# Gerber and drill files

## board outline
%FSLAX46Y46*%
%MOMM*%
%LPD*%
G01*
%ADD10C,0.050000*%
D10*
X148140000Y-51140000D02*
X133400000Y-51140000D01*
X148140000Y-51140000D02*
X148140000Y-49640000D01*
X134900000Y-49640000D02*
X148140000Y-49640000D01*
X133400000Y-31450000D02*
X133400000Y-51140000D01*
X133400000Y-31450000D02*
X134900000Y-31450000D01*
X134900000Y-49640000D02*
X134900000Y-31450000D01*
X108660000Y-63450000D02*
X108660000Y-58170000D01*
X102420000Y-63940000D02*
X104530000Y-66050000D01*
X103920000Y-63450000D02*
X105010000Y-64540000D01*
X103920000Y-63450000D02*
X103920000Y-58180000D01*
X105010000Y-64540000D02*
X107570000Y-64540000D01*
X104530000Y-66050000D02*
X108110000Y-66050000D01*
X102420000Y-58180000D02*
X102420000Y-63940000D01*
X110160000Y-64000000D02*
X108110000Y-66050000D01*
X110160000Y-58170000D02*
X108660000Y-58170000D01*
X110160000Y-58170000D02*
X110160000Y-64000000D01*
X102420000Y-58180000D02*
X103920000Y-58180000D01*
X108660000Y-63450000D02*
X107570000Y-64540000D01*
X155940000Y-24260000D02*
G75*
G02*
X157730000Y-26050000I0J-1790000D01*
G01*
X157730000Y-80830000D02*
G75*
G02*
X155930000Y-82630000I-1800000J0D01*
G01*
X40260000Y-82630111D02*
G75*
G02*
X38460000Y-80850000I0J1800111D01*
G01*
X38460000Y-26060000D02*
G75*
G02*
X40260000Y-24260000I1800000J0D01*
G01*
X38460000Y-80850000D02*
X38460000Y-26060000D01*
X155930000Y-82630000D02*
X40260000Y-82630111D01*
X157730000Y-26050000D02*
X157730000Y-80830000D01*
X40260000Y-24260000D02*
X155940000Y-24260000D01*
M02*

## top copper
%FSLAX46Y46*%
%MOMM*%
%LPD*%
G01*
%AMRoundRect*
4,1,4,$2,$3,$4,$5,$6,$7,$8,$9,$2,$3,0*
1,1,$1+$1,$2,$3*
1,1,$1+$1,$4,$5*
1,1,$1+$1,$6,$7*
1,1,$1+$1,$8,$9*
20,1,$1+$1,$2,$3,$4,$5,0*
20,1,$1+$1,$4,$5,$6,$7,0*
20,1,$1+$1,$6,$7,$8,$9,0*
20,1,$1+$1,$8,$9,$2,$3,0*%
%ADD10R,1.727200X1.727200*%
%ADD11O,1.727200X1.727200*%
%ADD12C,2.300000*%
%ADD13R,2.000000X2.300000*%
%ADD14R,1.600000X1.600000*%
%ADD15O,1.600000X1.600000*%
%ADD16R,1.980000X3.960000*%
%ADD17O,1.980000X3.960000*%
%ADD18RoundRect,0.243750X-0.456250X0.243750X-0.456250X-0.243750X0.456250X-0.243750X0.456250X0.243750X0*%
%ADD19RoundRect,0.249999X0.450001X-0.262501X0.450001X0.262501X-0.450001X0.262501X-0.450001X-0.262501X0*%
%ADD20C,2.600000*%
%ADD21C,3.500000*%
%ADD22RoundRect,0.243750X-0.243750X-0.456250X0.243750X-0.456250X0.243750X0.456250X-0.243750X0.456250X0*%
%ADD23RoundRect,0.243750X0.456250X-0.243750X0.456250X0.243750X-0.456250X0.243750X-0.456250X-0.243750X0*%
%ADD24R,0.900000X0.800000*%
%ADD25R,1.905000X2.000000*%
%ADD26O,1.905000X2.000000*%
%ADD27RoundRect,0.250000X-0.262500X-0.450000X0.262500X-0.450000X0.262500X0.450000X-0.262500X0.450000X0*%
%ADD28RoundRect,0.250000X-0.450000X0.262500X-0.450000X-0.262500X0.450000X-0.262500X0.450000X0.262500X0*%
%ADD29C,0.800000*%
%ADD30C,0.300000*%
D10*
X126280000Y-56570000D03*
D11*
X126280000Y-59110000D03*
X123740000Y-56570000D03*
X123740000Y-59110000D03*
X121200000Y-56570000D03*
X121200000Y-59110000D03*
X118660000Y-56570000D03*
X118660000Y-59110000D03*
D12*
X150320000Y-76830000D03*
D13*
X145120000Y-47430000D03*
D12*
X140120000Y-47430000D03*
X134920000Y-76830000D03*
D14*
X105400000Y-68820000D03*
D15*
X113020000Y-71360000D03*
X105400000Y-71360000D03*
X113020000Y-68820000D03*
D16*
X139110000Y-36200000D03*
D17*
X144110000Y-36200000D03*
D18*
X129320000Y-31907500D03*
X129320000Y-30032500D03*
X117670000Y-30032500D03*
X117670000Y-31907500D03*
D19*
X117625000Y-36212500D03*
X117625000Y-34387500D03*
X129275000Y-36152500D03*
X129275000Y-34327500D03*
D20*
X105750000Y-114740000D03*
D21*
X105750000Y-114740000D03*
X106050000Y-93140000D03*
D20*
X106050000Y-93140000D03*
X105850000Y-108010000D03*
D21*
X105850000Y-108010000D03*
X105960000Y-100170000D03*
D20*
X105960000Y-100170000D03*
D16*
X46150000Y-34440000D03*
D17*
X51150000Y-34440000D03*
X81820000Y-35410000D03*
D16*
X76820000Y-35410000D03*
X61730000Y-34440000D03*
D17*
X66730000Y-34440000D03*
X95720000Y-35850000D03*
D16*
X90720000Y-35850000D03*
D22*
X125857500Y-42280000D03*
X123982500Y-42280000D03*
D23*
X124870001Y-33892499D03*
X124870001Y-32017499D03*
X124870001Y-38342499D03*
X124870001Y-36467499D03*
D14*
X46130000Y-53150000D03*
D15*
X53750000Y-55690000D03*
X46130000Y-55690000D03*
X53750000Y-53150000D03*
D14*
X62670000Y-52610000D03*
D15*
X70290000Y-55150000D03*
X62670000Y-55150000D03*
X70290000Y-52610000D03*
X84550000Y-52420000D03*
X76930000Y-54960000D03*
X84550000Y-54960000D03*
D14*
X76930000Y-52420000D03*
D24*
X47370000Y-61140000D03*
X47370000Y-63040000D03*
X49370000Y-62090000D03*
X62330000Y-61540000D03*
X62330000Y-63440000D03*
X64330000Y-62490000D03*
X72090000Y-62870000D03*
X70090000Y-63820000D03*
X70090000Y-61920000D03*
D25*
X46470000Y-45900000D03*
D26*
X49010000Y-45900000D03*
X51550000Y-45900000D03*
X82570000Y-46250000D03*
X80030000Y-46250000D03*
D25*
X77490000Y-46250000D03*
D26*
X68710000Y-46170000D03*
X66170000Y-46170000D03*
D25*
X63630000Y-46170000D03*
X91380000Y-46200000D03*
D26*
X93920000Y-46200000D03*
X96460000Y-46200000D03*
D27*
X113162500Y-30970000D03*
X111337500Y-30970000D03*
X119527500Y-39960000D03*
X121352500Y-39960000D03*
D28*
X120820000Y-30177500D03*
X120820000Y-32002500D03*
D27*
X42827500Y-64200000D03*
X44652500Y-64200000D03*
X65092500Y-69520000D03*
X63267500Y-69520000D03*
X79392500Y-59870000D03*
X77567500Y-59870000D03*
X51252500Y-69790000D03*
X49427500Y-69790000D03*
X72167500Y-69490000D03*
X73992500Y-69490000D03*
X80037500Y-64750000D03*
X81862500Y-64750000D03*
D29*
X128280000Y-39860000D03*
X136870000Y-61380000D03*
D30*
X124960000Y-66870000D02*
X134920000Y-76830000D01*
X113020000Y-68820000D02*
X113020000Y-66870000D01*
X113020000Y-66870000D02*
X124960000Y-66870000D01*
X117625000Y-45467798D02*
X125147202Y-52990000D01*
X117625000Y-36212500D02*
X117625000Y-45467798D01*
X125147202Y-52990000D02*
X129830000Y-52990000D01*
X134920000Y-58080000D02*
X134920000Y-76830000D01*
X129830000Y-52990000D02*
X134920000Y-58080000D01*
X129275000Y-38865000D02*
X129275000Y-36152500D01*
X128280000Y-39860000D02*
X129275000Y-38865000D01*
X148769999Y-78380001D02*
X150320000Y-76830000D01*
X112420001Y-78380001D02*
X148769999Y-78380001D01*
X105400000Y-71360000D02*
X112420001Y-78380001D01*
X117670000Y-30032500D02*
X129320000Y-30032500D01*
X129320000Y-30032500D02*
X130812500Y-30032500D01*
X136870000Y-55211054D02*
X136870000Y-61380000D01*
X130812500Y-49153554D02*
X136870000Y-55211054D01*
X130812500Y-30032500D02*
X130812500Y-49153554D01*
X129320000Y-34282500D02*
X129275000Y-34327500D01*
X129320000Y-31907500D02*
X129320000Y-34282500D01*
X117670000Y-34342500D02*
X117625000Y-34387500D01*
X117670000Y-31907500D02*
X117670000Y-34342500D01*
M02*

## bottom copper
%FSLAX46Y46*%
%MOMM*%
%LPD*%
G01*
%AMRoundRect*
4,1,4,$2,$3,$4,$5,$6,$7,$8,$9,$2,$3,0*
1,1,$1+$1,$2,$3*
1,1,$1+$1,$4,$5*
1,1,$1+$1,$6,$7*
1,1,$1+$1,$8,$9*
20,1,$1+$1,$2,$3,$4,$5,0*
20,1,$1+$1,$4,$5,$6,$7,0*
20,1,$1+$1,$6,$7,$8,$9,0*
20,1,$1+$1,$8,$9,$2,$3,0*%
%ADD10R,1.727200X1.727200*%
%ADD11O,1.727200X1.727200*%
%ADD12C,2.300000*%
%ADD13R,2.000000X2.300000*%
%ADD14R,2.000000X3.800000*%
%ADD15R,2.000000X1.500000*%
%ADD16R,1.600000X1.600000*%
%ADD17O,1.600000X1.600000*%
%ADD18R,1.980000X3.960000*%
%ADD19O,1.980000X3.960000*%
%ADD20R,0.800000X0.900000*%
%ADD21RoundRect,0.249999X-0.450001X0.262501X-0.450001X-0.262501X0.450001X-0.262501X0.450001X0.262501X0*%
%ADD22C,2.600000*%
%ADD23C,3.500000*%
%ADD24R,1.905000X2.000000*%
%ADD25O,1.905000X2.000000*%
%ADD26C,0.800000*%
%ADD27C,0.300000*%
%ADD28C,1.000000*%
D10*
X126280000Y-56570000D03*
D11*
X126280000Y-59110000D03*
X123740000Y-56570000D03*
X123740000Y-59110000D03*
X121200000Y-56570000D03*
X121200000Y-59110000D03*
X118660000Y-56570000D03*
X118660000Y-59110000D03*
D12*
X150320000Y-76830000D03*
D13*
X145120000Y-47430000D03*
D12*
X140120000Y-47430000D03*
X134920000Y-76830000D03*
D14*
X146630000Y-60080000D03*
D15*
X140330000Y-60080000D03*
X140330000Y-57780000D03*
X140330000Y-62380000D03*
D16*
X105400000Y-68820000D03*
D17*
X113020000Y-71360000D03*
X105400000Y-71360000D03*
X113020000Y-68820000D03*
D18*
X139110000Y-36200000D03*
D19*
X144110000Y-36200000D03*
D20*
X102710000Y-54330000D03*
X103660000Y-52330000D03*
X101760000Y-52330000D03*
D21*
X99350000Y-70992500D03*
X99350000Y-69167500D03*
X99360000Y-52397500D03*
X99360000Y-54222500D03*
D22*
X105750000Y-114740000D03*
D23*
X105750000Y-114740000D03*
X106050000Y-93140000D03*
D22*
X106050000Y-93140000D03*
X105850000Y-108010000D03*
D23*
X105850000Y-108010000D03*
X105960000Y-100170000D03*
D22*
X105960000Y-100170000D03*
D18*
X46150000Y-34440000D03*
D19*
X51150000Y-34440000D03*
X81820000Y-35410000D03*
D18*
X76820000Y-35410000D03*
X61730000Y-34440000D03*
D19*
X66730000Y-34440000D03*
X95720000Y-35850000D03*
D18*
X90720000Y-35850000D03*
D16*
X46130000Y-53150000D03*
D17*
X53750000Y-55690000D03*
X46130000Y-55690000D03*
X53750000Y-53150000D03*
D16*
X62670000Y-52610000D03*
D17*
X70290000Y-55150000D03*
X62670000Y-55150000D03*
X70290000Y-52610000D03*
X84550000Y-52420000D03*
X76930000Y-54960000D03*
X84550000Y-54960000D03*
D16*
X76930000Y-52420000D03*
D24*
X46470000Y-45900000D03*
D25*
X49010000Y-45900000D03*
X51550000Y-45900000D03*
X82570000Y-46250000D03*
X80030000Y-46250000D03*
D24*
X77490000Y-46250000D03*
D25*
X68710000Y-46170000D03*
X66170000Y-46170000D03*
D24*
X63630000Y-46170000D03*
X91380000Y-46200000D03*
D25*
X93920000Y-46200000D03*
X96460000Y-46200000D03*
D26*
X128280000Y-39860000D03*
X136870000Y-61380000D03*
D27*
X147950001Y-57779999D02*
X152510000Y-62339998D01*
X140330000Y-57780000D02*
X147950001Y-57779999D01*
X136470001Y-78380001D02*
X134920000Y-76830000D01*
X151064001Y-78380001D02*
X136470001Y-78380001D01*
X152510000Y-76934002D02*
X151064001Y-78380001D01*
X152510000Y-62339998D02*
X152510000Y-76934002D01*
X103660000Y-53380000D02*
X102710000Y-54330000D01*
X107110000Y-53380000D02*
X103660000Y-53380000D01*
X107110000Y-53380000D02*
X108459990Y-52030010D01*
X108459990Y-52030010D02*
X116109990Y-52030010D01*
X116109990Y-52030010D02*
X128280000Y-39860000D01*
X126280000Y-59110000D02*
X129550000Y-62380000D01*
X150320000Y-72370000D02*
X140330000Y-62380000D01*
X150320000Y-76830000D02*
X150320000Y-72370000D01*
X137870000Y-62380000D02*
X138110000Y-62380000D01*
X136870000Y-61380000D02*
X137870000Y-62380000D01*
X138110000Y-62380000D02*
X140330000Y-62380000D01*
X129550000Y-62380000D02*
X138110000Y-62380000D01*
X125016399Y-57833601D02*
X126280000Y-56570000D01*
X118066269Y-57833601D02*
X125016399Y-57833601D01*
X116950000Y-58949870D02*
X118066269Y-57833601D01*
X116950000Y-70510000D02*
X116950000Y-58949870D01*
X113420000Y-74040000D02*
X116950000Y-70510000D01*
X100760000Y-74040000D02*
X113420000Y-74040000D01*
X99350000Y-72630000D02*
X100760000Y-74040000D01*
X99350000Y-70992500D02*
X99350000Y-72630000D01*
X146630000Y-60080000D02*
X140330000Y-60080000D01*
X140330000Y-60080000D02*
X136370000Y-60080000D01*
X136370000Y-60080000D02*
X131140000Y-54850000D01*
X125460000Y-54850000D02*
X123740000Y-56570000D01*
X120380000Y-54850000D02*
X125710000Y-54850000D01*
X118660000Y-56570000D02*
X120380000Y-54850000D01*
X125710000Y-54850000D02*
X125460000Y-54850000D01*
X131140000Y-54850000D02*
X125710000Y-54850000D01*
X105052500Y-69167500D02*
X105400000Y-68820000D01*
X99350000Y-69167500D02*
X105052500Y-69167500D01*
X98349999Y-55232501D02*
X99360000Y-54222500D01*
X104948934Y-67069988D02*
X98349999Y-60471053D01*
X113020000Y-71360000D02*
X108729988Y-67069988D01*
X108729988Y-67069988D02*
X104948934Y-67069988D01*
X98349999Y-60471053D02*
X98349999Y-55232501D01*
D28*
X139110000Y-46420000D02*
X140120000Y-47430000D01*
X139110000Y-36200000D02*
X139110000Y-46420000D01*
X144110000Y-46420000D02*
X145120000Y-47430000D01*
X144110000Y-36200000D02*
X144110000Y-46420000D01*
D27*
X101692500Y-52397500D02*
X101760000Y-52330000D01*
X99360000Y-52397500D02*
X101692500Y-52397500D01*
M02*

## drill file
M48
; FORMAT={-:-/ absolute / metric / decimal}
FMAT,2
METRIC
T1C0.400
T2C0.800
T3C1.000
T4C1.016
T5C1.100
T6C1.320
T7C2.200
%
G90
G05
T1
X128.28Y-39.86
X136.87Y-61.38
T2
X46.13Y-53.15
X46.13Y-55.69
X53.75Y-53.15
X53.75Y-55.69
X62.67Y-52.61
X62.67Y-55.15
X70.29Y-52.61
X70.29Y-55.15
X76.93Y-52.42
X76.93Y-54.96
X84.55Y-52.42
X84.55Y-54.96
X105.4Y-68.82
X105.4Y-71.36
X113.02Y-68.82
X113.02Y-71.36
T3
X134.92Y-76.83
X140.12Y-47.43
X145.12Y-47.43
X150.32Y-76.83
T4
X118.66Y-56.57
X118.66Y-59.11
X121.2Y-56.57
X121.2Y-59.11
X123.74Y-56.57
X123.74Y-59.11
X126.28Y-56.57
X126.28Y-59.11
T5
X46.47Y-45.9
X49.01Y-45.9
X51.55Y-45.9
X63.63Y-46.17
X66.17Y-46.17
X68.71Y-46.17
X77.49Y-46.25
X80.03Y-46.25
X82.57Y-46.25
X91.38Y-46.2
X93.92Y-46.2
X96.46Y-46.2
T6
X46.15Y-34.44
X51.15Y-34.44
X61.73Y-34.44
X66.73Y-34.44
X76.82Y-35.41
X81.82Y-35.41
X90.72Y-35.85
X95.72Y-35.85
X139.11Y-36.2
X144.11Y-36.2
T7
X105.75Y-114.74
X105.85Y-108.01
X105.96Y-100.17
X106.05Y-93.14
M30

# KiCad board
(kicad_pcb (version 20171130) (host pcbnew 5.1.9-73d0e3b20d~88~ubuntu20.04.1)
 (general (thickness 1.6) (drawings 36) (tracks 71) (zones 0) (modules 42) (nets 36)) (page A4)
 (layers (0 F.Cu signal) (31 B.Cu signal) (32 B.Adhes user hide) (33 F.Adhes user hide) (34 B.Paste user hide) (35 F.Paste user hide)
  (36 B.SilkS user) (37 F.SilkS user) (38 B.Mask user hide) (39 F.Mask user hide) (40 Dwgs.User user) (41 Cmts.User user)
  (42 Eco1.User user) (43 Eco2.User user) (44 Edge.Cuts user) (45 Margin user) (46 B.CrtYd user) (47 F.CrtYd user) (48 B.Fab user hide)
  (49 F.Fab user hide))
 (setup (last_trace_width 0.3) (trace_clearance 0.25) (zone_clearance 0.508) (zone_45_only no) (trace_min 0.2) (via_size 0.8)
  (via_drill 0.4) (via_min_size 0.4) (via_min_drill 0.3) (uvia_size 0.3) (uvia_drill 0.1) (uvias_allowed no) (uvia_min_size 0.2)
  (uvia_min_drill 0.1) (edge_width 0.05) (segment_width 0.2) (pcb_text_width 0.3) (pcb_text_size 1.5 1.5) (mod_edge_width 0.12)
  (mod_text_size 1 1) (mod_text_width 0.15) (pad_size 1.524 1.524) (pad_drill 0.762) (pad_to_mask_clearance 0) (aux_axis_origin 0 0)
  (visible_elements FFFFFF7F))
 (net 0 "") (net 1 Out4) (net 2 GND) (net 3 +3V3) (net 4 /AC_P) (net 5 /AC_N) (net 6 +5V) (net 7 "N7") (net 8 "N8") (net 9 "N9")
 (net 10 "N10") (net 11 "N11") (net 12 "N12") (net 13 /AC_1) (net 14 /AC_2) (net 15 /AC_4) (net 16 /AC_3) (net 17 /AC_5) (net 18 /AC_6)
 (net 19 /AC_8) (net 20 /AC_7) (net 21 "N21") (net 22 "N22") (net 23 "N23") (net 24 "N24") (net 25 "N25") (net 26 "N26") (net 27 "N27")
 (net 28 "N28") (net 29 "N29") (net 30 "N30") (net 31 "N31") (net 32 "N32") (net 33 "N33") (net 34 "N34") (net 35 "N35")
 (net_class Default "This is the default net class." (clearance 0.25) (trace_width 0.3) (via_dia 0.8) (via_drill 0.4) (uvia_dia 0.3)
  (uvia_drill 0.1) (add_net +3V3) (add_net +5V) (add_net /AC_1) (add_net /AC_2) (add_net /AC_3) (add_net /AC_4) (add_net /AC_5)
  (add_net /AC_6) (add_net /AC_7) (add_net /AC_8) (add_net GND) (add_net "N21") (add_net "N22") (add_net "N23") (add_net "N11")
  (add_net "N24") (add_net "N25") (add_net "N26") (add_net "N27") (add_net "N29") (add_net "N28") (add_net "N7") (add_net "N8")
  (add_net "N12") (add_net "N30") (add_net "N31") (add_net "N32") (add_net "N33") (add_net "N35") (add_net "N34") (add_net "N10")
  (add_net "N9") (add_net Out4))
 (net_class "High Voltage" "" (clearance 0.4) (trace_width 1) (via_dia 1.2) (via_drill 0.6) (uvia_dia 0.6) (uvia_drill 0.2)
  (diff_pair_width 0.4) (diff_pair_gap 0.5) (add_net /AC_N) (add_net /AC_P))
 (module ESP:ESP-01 (layer F.Cu) (at 126.28 56.57 270)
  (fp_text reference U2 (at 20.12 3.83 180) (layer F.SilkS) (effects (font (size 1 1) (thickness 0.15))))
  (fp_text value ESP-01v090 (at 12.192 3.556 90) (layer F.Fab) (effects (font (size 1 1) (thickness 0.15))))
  (pad 1 thru_hole rect (at 0 0 270) (size 1.7272 1.7272) (drill 1.016) (layers *.Cu *.Mask F.SilkS) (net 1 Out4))
  (pad 2 thru_hole oval (at 2.54 0 270) (size 1.7272 1.7272) (drill 1.016) (layers *.Cu *.Mask F.SilkS) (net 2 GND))
  (pad 3 thru_hole oval (at 0 2.54 270) (size 1.7272 1.7272) (drill 1.016) (layers *.Cu *.Mask F.SilkS) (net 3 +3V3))
  (pad 4 thru_hole oval (at 2.54 2.54 270) (size 1.7272 1.7272) (drill 1.016) (layers *.Cu *.Mask F.SilkS))
  (pad 5 thru_hole oval (at 0 5.08 270) (size 1.7272 1.7272) (drill 1.016) (layers *.Cu *.Mask F.SilkS))
  (pad 6 thru_hole oval (at 2.54 5.08 270) (size 1.7272 1.7272) (drill 1.016) (layers *.Cu *.Mask F.SilkS))
  (pad 7 thru_hole oval (at 0 7.62 270) (size 1.7272 1.7272) (drill 1.016) (layers *.Cu *.Mask F.SilkS) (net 3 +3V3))
  (pad 8 thru_hole oval (at 2.54 7.62 270) (size 1.7272 1.7272) (drill 1.016) (layers *.Cu *.Mask F.SilkS)))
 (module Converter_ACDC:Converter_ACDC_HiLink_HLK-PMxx (layer F.Cu) (at 145.12 47.43 270)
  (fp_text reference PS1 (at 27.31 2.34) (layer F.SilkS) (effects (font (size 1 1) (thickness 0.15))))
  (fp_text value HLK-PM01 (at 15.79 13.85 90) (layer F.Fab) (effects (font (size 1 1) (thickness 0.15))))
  (pad 3 thru_hole circle (at 29.4 -5.2 270) (size 2.3 2.3) (drill 1) (layers *.Cu *.Mask) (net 2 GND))
  (pad 1 thru_hole rect (at 0 0 270) (size 2.3 2) (drill 1) (layers *.Cu *.Mask) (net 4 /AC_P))
  (pad 2 thru_hole circle (at 0 5 270) (size 2.3 2.3) (drill 1) (layers *.Cu *.Mask) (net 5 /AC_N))
  (pad 4 thru_hole circle (at 29.4 10.2 270) (size 2.3 2.3) (drill 1) (layers *.Cu *.Mask) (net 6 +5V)))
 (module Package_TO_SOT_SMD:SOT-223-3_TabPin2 (layer B.Cu) (at 143.48 60.08)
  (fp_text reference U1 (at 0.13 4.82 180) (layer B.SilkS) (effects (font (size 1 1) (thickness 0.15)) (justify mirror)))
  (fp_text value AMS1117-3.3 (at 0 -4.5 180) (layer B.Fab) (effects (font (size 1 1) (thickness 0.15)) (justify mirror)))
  (pad 2 smd rect (at 3.15 0) (size 2 3.8) (layers B.Cu B.Paste B.Mask) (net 3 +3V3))
  (pad 2 smd rect (at -3.15 0) (size 2 1.5) (layers B.Cu B.Paste B.Mask) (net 3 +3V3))
  (pad 3 smd rect (at -3.15 -2.3) (size 2 1.5) (layers B.Cu B.Paste B.Mask) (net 6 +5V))
  (pad 1 smd rect (at -3.15 2.3) (size 2 1.5) (layers B.Cu B.Paste B.Mask) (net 2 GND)))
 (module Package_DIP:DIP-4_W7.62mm (layer F.Cu) (at 105.4 68.82)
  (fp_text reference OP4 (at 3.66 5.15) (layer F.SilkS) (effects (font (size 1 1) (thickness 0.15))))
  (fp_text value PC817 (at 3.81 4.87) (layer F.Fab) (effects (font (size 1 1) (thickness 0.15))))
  (pad 1 thru_hole rect (at 0 0) (size 1.6 1.6) (drill 0.8) (layers *.Cu *.Mask) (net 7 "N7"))
  (pad 3 thru_hole oval (at 7.62 2.54) (size 1.6 1.6) (drill 0.8) (layers *.Cu *.Mask) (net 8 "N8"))
  (pad 2 thru_hole oval (at 0 2.54) (size 1.6 1.6) (drill 0.8) (layers *.Cu *.Mask) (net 2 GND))
  (pad 4 thru_hole oval (at 7.62 0) (size 1.6 1.6) (drill 0.8) (layers *.Cu *.Mask) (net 6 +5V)))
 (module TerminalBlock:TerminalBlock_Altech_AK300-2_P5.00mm (layer F.Cu) (at 139.11 36.2)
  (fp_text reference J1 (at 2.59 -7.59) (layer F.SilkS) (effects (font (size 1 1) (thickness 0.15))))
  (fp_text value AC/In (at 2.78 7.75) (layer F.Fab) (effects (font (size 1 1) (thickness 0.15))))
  (pad 1 thru_hole rect (at 0 0) (size 1.98 3.96) (drill 1.32) (layers *.Cu *.Mask) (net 5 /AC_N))
  (pad 2 thru_hole oval (at 5 0) (size 1.98 3.96) (drill 1.32) (layers *.Cu *.Mask) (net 4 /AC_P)))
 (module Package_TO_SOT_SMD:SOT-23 (layer B.Cu) (at 102.71 53.33 270)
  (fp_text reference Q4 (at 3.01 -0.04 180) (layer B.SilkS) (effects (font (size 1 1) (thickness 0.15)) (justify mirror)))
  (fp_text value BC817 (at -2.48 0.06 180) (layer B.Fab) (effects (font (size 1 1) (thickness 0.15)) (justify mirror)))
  (pad 3 smd rect (at 1 0 270) (size 0.9 0.8) (layers B.Cu B.Paste B.Mask) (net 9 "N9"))
  (pad 2 smd rect (at -1 -0.95 270) (size 0.9 0.8) (layers B.Cu B.Paste B.Mask) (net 2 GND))
  (pad 1 smd rect (at -1 0.95 270) (size 0.9 0.8) (layers B.Cu B.Paste B.Mask) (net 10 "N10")))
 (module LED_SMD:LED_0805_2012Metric (layer F.Cu) (at 129.32 30.97 270)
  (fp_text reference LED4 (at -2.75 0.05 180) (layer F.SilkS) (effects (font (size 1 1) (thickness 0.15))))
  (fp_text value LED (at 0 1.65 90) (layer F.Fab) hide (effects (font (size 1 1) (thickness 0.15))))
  (pad 2 smd roundrect (at 0.9375 0 270) (size 0.975 1.4) (layers F.Cu F.Paste F.Mask) (roundrect_rratio 0.25) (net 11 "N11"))
  (pad 1 smd roundrect (at -0.9375 0 270) (size 0.975 1.4) (layers F.Cu F.Paste F.Mask) (roundrect_rratio 0.25) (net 2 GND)))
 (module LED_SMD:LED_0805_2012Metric (layer F.Cu) (at 117.67 30.97 270)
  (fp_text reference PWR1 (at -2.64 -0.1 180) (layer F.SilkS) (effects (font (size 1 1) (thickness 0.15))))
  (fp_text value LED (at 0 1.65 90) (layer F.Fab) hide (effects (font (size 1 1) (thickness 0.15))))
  (pad 1 smd roundrect (at -0.9375 0 270) (size 0.975 1.4) (layers F.Cu F.Paste F.Mask) (roundrect_rratio 0.25) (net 2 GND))
  (pad 2 smd roundrect (at 0.9375 0 270) (size 0.975 1.4) (layers F.Cu F.Paste F.Mask) (roundrect_rratio 0.25) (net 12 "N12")))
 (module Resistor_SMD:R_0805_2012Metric (layer F.Cu) (at 117.625 35.3 90)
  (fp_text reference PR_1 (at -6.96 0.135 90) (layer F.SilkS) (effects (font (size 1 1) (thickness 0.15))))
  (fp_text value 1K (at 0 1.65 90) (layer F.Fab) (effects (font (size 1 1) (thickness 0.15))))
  (pad 1 smd roundrect (at -0.9125 0 90) (size 1.025 1.4) (layers F.Cu F.Paste F.Mask) (roundrect_rratio 0.2439014634146341) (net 6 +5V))
  (pad 2 smd roundrect (at 0.9125 0 90) (size 1.025 1.4) (layers F.Cu F.Paste F.Mask) (roundrect_rratio 0.2439014634146341) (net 12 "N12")))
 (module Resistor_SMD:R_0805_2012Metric (layer F.Cu) (at 129.275 35.24 90)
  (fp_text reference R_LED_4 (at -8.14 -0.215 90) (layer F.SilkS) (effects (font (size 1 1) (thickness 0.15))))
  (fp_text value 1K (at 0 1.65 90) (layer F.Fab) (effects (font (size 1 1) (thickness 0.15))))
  (pad 1 smd roundrect (at -0.9125 0 90) (size 1.025 1.4) (layers F.Cu F.Paste F.Mask) (roundrect_rratio 0.2439014634146341) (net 9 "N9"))
  (pad 2 smd roundrect (at 0.9125 0 90) (size 1.025 1.4) (layers F.Cu F.Paste F.Mask) (roundrect_rratio 0.2439014634146341) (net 11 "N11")))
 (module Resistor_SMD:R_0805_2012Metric (layer B.Cu) (at 99.35 70.08 270)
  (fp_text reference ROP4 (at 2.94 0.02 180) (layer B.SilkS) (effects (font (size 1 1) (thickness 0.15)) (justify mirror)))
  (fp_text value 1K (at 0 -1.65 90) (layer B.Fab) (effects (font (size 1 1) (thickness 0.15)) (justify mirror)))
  (pad 2 smd roundrect (at 0.9125 0 270) (size 1.025 1.4) (layers B.Cu B.Paste B.Mask) (roundrect_rratio 0.2439014634146341) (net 1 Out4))
  (pad 1 smd roundrect (at -0.9125 0 270) (size 1.025 1.4) (layers B.Cu B.Paste B.Mask) (roundrect_rratio 0.2439014634146341) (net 7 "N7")))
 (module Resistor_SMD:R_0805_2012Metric (layer B.Cu) (at 99.36 53.31 270)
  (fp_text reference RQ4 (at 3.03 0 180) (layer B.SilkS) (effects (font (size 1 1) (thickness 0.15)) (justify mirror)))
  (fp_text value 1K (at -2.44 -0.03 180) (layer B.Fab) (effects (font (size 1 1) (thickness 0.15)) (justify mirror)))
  (pad 1 smd roundrect (at -0.9125 0 270) (size 1.025 1.4) (layers B.Cu B.Paste B.Mask) (roundrect_rratio 0.2439014634146341) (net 10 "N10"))
  (pad 2 smd roundrect (at 0.9125 0 270) (size 1.025 1.4) (layers B.Cu B.Paste B.Mask) (roundrect_rratio 0.2439014634146341) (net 8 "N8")))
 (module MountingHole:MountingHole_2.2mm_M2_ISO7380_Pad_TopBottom (layer F.Cu) (at 105.75 114.74)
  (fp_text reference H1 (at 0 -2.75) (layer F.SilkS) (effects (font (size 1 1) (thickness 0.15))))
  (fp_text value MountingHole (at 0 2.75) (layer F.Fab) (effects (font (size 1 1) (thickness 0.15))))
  (pad 1 thru_hole circle (at 0 0) (size 2.6 2.6) (drill 2.2) (layers *.Cu *.Mask))
  (pad 1 connect circle (at 0 0) (size 3.5 3.5) (layers F.Cu F.Mask))
  (pad 1 connect circle (at 0 0) (size 3.5 3.5) (layers B.Cu B.Mask)))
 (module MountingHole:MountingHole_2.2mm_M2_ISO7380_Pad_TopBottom (layer F.Cu) (at 106.05 93.14)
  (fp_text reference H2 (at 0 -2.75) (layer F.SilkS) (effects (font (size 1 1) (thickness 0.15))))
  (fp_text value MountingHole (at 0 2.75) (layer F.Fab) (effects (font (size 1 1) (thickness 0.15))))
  (pad 1 connect circle (at 0 0) (size 3.5 3.5) (layers B.Cu B.Mask))
  (pad 1 connect circle (at 0 0) (size 3.5 3.5) (layers F.Cu F.Mask))
  (pad 1 thru_hole circle (at 0 0) (size 2.6 2.6) (drill 2.2) (layers *.Cu *.Mask)))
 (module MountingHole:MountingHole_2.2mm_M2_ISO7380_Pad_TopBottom (layer F.Cu) (at 105.85 108.01)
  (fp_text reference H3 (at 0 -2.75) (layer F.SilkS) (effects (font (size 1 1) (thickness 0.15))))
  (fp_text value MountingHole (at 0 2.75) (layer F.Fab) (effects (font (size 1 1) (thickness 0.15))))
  (pad 1 thru_hole circle (at 0 0) (size 2.6 2.6) (drill 2.2) (layers *.Cu *.Mask))
  (pad 1 connect circle (at 0 0) (size 3.5 3.5) (layers F.Cu F.Mask))
  (pad 1 connect circle (at 0 0) (size 3.5 3.5) (layers B.Cu B.Mask)))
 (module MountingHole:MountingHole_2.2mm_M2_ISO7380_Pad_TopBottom (layer F.Cu) (at 105.96 100.17)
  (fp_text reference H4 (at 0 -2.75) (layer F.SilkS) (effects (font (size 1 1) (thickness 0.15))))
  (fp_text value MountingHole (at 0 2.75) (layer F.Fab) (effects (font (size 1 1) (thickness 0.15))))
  (pad 1 connect circle (at 0 0) (size 3.5 3.5) (layers B.Cu B.Mask))
  (pad 1 connect circle (at 0 0) (size 3.5 3.5) (layers F.Cu F.Mask))
  (pad 1 thru_hole circle (at 0 0) (size 2.6 2.6) (drill 2.2) (layers *.Cu *.Mask)))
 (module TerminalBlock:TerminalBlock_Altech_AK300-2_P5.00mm (layer F.Cu) (at 46.15 34.44)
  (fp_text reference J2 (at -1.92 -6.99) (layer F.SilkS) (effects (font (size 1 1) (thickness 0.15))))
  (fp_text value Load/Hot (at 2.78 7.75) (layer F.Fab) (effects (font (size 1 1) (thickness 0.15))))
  (pad 1 thru_hole rect (at 0 0) (size 1.98 3.96) (drill 1.32) (layers *.Cu *.Mask) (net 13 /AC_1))
  (pad 2 thru_hole oval (at 5 0) (size 1.98 3.96) (drill 1.32) (layers *.Cu *.Mask) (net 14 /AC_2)))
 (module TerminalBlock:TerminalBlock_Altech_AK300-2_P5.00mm (layer F.Cu) (at 76.82 35.41)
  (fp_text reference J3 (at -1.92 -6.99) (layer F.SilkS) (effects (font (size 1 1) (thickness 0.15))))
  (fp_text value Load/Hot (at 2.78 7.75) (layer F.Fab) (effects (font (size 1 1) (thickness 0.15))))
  (pad 2 thru_hole oval (at 5 0) (size 1.98 3.96) (drill 1.32) (layers *.Cu *.Mask) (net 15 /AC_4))
  (pad 1 thru_hole rect (at 0 0) (size 1.98 3.96) (drill 1.32) (layers *.Cu *.Mask) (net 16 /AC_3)))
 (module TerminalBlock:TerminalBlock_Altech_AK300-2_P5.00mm (layer F.Cu) (at 61.73 34.44)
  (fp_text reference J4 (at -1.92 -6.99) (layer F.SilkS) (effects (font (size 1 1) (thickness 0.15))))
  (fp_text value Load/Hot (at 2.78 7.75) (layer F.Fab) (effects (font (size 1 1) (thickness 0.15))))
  (pad 1 thru_hole rect (at 0 0) (size 1.98 3.96) (drill 1.32) (layers *.Cu *.Mask) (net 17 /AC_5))
  (pad 2 thru_hole oval (at 5 0) (size 1.98 3.96) (drill 1.32) (layers *.Cu *.Mask) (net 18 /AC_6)))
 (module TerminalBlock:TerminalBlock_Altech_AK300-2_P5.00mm (layer F.Cu) (at 90.72 35.85)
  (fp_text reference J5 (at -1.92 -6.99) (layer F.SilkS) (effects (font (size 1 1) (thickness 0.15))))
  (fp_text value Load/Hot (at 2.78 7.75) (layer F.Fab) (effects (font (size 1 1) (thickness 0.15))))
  (pad 2 thru_hole oval (at 5 0) (size 1.98 3.96) (drill 1.32) (layers *.Cu *.Mask) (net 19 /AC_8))
  (pad 1 thru_hole rect (at 0 0) (size 1.98 3.96) (drill 1.32) (layers *.Cu *.Mask) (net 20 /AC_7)))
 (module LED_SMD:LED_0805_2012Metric (layer F.Cu) (at 124.92 42.28)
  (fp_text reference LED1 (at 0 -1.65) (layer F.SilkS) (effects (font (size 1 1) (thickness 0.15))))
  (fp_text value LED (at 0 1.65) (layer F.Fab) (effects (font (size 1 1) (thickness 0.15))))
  (pad 2 smd roundrect (at 0.9375 0) (size 0.975 1.4) (layers F.Cu F.Paste F.Mask) (roundrect_rratio 0.25) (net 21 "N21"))
  (pad 1 smd roundrect (at -0.9375 0) (size 0.975 1.4) (layers F.Cu F.Paste F.Mask) (roundrect_rratio 0.25) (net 2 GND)))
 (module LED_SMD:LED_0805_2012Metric (layer F.Cu) (at 124.870001 32.954999 90)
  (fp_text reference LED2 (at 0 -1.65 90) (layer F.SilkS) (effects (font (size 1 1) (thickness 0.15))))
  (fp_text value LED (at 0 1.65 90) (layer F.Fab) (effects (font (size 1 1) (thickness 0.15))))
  (pad 1 smd roundrect (at -0.9375 0 90) (size 0.975 1.4) (layers F.Cu F.Paste F.Mask) (roundrect_rratio 0.25) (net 2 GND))
  (pad 2 smd roundrect (at 0.9375 0 90) (size 0.975 1.4) (layers F.Cu F.Paste F.Mask) (roundrect_rratio 0.25) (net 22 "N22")))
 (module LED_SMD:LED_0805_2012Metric (layer F.Cu) (at 124.870001 37.404999 90)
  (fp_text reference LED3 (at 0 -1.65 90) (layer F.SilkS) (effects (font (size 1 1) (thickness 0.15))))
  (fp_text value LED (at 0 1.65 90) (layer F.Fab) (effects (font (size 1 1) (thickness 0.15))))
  (pad 1 smd roundrect (at -0.9375 0 90) (size 0.975 1.4) (layers F.Cu F.Paste F.Mask) (roundrect_rratio 0.25) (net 2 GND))
  (pad 2 smd roundrect (at 0.9375 0 90) (size 0.975 1.4) (layers F.Cu F.Paste F.Mask) (roundrect_rratio 0.25) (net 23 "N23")))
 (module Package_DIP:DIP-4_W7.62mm (layer F.Cu) (at 46.13 53.15)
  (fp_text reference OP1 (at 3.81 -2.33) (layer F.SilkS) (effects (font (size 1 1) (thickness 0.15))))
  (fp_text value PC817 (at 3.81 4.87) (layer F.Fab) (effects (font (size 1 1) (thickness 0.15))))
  (pad 1 thru_hole rect (at 0 0) (size 1.6 1.6) (drill 0.8) (layers *.Cu *.Mask) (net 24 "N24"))
  (pad 3 thru_hole oval (at 7.62 2.54) (size 1.6 1.6) (drill 0.8) (layers *.Cu *.Mask) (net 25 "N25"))
  (pad 2 thru_hole oval (at 0 2.54) (size 1.6 1.6) (drill 0.8) (layers *.Cu *.Mask) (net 2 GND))
  (pad 4 thru_hole oval (at 7.62 0) (size 1.6 1.6) (drill 0.8) (layers *.Cu *.Mask) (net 6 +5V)))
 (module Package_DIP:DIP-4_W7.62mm (layer F.Cu) (at 62.67 52.61)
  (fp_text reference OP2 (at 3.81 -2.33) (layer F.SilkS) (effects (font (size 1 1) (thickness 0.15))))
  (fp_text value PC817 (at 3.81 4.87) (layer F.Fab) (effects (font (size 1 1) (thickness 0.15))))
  (pad 1 thru_hole rect (at 0 0) (size 1.6 1.6) (drill 0.8) (layers *.Cu *.Mask) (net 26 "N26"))
  (pad 3 thru_hole oval (at 7.62 2.54) (size 1.6 1.6) (drill 0.8) (layers *.Cu *.Mask) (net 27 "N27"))
  (pad 2 thru_hole oval (at 0 2.54) (size 1.6 1.6) (drill 0.8) (layers *.Cu *.Mask) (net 2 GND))
  (pad 4 thru_hole oval (at 7.62 0) (size 1.6 1.6) (drill 0.8) (layers *.Cu *.Mask) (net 6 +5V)))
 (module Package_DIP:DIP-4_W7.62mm (layer F.Cu) (at 76.93 52.42)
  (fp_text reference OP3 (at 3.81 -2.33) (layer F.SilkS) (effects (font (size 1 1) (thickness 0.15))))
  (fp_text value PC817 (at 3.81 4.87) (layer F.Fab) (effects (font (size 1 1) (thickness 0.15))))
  (pad 4 thru_hole oval (at 7.62 0) (size 1.6 1.6) (drill 0.8) (layers *.Cu *.Mask) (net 6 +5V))
  (pad 2 thru_hole oval (at 0 2.54) (size 1.6 1.6) (drill 0.8) (layers *.Cu *.Mask) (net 2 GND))
  (pad 3 thru_hole oval (at 7.62 2.54) (size 1.6 1.6) (drill 0.8) (layers *.Cu *.Mask) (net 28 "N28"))
  (pad 1 thru_hole rect (at 0 0) (size 1.6 1.6) (drill 0.8) (layers *.Cu *.Mask) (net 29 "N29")))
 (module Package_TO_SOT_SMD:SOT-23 (layer F.Cu) (at 48.37 62.09)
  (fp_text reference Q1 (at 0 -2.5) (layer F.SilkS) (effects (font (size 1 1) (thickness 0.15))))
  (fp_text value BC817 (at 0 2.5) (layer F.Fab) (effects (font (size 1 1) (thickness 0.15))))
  (pad 1 smd rect (at -1 -0.95) (size 0.9 0.8) (layers F.Cu F.Paste F.Mask) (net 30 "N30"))
  (pad 2 smd rect (at -1 0.95) (size 0.9 0.8) (layers F.Cu F.Paste F.Mask) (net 2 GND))
  (pad 3 smd rect (at 1 0) (size 0.9 0.8) (layers F.Cu F.Paste F.Mask) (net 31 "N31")))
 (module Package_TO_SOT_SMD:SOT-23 (layer F.Cu) (at 63.33 62.49)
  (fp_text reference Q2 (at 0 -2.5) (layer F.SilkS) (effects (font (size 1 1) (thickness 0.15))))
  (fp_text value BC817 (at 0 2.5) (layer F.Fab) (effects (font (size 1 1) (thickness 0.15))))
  (pad 1 smd rect (at -1 -0.95) (size 0.9 0.8) (layers F.Cu F.Paste F.Mask) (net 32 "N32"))
  (pad 2 smd rect (at -1 0.95) (size 0.9 0.8) (layers F.Cu F.Paste F.Mask) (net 2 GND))
  (pad 3 smd rect (at 1 0) (size 0.9 0.8) (layers F.Cu F.Paste F.Mask) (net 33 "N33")))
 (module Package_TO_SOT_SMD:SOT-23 (layer F.Cu) (at 71.09 62.87)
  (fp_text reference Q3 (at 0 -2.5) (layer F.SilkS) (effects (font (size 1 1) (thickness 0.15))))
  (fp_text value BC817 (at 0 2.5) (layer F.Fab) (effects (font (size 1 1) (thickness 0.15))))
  (pad 3 smd rect (at 1 0) (size 0.9 0.8) (layers F.Cu F.Paste F.Mask) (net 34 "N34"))
  (pad 2 smd rect (at -1 0.95) (size 0.9 0.8) (layers F.Cu F.Paste F.Mask) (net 2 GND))
  (pad 1 smd rect (at -1 -0.95) (size 0.9 0.8) (layers F.Cu F.Paste F.Mask) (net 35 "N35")))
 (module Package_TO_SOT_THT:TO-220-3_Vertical (layer F.Cu) (at 46.47 45.9)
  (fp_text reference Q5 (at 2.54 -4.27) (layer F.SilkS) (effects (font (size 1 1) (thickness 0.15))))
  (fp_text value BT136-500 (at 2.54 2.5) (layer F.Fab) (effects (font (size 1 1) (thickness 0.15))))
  (pad 1 thru_hole rect (at 0 0) (size 1.905 2) (drill 1.1) (layers *.Cu *.Mask) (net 13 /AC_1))
  (pad 2 thru_hole oval (at 2.54 0) (size 1.905 2) (drill 1.1) (layers *.Cu *.Mask) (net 14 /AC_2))
  (pad 3 thru_hole oval (at 5.08 0) (size 1.905 2) (drill 1.1) (layers *.Cu *.Mask) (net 31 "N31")))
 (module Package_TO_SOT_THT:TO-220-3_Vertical (layer F.Cu) (at 77.49 46.25)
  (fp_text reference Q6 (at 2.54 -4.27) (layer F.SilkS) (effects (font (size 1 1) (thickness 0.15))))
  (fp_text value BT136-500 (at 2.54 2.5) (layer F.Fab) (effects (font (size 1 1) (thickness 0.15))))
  (pad 3 thru_hole oval (at 5.08 0) (size 1.905 2) (drill 1.1) (layers *.Cu *.Mask) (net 33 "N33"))
  (pad 2 thru_hole oval (at 2.54 0) (size 1.905 2) (drill 1.1) (layers *.Cu *.Mask) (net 15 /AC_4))
  (pad 1 thru_hole rect (at 0 0) (size 1.905 2) (drill 1.1) (layers *.Cu *.Mask) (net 16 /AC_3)))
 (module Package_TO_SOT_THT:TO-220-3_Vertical (layer F.Cu) (at 63.63 46.17)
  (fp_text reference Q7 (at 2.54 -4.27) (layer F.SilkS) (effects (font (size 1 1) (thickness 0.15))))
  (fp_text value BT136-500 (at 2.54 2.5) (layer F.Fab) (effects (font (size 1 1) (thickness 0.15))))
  (pad 3 thru_hole oval (at 5.08 0) (size 1.905 2) (drill 1.1) (layers *.Cu *.Mask) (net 34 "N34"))
  (pad 2 thru_hole oval (at 2.54 0) (size 1.905 2) (drill 1.1) (layers *.Cu *.Mask) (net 18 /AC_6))
  (pad 1 thru_hole rect (at 0 0) (size 1.905 2) (drill 1.1) (layers *.Cu *.Mask) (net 17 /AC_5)))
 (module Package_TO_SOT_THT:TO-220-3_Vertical (layer F.Cu) (at 91.38 46.2)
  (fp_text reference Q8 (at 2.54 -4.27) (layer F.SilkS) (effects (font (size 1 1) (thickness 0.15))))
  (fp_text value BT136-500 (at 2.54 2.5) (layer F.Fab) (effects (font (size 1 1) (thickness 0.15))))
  (pad 1 thru_hole rect (at 0 0) (size 1.905 2) (drill 1.1) (layers *.Cu *.Mask) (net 20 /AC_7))
  (pad 2 thru_hole oval (at 2.54 0) (size 1.905 2) (drill 1.1) (layers *.Cu *.Mask) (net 19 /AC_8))
  (pad 3 thru_hole oval (at 5.08 0) (size 1.905 2) (drill 1.1) (layers *.Cu *.Mask) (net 9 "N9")))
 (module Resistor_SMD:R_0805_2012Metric (layer F.Cu) (at 112.25 30.97)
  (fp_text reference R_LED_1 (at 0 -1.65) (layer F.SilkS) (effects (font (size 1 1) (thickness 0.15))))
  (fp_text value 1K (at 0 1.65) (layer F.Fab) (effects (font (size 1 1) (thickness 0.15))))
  (pad 2 smd roundrect (at 0.9125 0) (size 1.025 1.4) (layers F.Cu F.Paste F.Mask) (roundrect_rratio 0.243902) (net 21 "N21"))
  (pad 1 smd roundrect (at -0.9125 0) (size 1.025 1.4) (layers F.Cu F.Paste F.Mask) (roundrect_rratio 0.243902) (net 31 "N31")))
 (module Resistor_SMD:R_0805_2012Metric (layer F.Cu) (at 120.44 39.96)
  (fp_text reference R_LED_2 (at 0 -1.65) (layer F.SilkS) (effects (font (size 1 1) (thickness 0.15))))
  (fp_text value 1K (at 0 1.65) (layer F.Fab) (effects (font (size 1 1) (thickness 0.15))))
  (pad 1 smd roundrect (at -0.9125 0) (size 1.025 1.4) (layers F.Cu F.Paste F.Mask) (roundrect_rratio 0.243902) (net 33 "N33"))
  (pad 2 smd roundrect (at 0.9125 0) (size 1.025 1.4) (layers F.Cu F.Paste F.Mask) (roundrect_rratio 0.243902) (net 22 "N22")))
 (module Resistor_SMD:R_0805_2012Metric (layer F.Cu) (at 120.82 31.09 270)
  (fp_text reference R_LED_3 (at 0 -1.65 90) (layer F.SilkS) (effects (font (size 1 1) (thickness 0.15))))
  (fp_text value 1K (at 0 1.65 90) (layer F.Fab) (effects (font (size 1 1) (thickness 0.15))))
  (pad 1 smd roundrect (at -0.9125 0 270) (size 1.025 1.4) (layers F.Cu F.Paste F.Mask) (roundrect_rratio 0.243902) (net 34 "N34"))
  (pad 2 smd roundrect (at 0.9125 0 270) (size 1.025 1.4) (layers F.Cu F.Paste F.Mask) (roundrect_rratio 0.243902) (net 23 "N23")))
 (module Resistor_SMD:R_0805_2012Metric (layer F.Cu) (at 43.74 64.2)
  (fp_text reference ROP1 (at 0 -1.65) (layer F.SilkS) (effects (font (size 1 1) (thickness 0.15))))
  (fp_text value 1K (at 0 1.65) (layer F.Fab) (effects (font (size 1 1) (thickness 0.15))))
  (pad 1 smd roundrect (at -0.9125 0) (size 1.025 1.4) (layers F.Cu F.Paste F.Mask) (roundrect_rratio 0.243902) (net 24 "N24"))
  (pad 2 smd roundrect (at 0.9125 0) (size 1.025 1.4) (layers F.Cu F.Paste F.Mask) (roundrect_rratio 0.243902) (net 1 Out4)))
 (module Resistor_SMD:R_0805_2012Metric (layer F.Cu) (at 64.18 69.52)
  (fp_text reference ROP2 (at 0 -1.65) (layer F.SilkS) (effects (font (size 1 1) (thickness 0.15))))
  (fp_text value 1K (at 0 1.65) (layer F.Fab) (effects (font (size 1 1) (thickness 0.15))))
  (pad 2 smd roundrect (at 0.9125 0) (size 1.025 1.4) (layers F.Cu F.Paste F.Mask) (roundrect_rratio 0.243902) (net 1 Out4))
  (pad 1 smd roundrect (at -0.9125 0) (size 1.025 1.4) (layers F.Cu F.Paste F.Mask) (roundrect_rratio 0.243902) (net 26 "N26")))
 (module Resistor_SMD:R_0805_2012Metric (layer F.Cu) (at 78.48 59.87)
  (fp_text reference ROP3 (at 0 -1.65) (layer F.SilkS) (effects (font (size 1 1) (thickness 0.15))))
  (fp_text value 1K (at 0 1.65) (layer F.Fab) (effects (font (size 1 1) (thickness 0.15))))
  (pad 2 smd roundrect (at 0.9125 0) (size 1.025 1.4) (layers F.Cu F.Paste F.Mask) (roundrect_rratio 0.243902) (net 1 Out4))
  (pad 1 smd roundrect (at -0.9125 0) (size 1.025 1.4) (layers F.Cu F.Paste F.Mask) (roundrect_rratio 0.243902) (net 29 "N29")))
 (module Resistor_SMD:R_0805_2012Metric (layer F.Cu) (at 50.34 69.79)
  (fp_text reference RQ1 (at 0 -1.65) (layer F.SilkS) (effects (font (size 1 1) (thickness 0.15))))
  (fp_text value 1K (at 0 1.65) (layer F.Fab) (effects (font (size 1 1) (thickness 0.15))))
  (pad 2 smd roundrect (at 0.9125 0) (size 1.025 1.4) (layers F.Cu F.Paste F.Mask) (roundrect_rratio 0.243902) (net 25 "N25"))
  (pad 1 smd roundrect (at -0.9125 0) (size 1.025 1.4) (layers F.Cu F.Paste F.Mask) (roundrect_rratio 0.243902) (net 30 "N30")))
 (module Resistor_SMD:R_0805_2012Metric (layer F.Cu) (at 73.08 69.49)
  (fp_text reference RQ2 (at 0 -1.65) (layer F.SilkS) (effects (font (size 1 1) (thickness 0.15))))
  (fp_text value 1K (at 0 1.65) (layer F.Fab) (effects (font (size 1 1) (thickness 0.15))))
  (pad 1 smd roundrect (at -0.9125 0) (size 1.025 1.4) (layers F.Cu F.Paste F.Mask) (roundrect_rratio 0.243902) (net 32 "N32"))
  (pad 2 smd roundrect (at 0.9125 0) (size 1.025 1.4) (layers F.Cu F.Paste F.Mask) (roundrect_rratio 0.243902) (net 27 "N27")))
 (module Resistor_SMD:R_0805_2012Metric (layer F.Cu) (at 80.95 64.75)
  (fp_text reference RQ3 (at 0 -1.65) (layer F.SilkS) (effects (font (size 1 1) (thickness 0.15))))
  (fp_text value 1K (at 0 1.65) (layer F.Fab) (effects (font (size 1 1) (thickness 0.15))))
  (pad 1 smd roundrect (at -0.9125 0) (size 1.025 1.4) (layers F.Cu F.Paste F.Mask) (roundrect_rratio 0.243902) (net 35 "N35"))
  (pad 2 smd roundrect (at 0.9125 0) (size 1.025 1.4) (layers F.Cu F.Paste F.Mask) (roundrect_rratio 0.243902) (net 28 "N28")))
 (gr_line (start 148.14 51.14) (end 133.4 51.14) (layer Edge.Cuts) (width 0.05))
 (gr_line (start 148.14 51.14) (end 148.14 49.64) (layer Edge.Cuts) (width 0.05))
 (gr_line (start 134.9 49.64) (end 148.14 49.64) (layer Edge.Cuts) (width 0.05))
 (gr_line (start 133.4 31.45) (end 133.4 51.14) (layer Edge.Cuts) (width 0.05))
 (gr_line (start 133.4 31.45) (end 134.9 31.45) (layer Edge.Cuts) (width 0.05))
 (gr_line (start 134.9 49.64) (end 134.9 31.45) (layer Edge.Cuts) (width 0.05))
 (gr_line (start 108.66 63.45) (end 108.66 58.17) (layer Edge.Cuts) (width 0.05))
 (gr_line (start 102.42 63.94) (end 104.53 66.05) (layer Edge.Cuts) (width 0.05))
 (gr_line (start 103.92 63.45) (end 105.01 64.54) (layer Edge.Cuts) (width 0.05))
 (gr_line (start 103.92 63.45) (end 103.92 58.18) (layer Edge.Cuts) (width 0.05))
 (gr_line (start 105.01 64.54) (end 107.57 64.54) (layer Edge.Cuts) (width 0.05))
 (gr_line (start 104.53 66.05) (end 108.11 66.05) (layer Edge.Cuts) (width 0.05))
 (gr_line (start 102.42 58.18) (end 102.42 63.94) (layer Edge.Cuts) (width 0.05))
 (gr_line (start 110.16 64) (end 108.11 66.05) (layer Edge.Cuts) (width 0.05))
 (gr_line (start 110.16 58.17) (end 108.66 58.17) (layer Edge.Cuts) (width 0.05))
 (gr_line (start 110.16 58.17) (end 110.16 64) (layer Edge.Cuts) (width 0.05))
 (gr_line (start 102.42 58.18) (end 103.92 58.18) (layer Edge.Cuts) (width 0.05))
 (gr_line (start 108.66 63.45) (end 107.57 64.54) (layer Edge.Cuts) (width 0.05))
 (gr_arc (start 155.94 26.05) (end 157.73 26.05) (angle -90) (layer Edge.Cuts) (width 0.05))
 (gr_arc (start 155.93 80.83) (end 155.93 82.63) (angle -90) (layer Edge.Cuts) (width 0.05))
 (gr_arc (start 40.26 80.83) (end 38.46 80.85) (angle -89.36340642) (layer Edge.Cuts) (width 0.05))
 (gr_arc (start 40.26 26.06) (end 40.26 24.26) (angle -90) (layer Edge.Cuts) (width 0.05))
 (gr_line (start 38.46 80.85) (end 38.46 26.06) (layer Edge.Cuts) (width 0.05))
 (gr_line (start 155.93 82.63) (end 40.26 82.630111) (layer Edge.Cuts) (width 0.05))
 (gr_line (start 157.73 26.05) (end 157.73 80.83) (layer Edge.Cuts) (width 0.05))
 (gr_line (start 40.26 24.26) (end 155.94 24.26) (layer Edge.Cuts) (width 0.05))
 (segment (start 124.96 66.87) (end 134.92 76.83) (width 0.3) (layer F.Cu) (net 6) (status 20))
 (segment (start 113.02 68.82) (end 113.02 66.87) (width 0.3) (layer F.Cu) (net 6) (status 10))
 (segment (start 113.02 66.87) (end 124.96 66.87) (width 0.3) (layer F.Cu) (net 6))
 (segment (start 147.950001 57.779999) (end 152.51 62.339998) (width 0.3) (layer B.Cu) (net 6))
 (segment (start 140.33 57.78) (end 147.950001 57.779999) (width 0.3) (layer B.Cu) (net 6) (status 10))
 (segment (start 136.470001 78.380001) (end 134.92 76.83) (width 0.3) (layer B.Cu) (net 6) (status 20))
 (segment (start 151.064001 78.380001) (end 136.470001 78.380001) (width 0.3) (layer B.Cu) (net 6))
 (segment (start 152.51 76.934002) (end 151.064001 78.380001) (width 0.3) (layer B.Cu) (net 6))
 (segment (start 152.51 62.339998) (end 152.51 76.934002) (width 0.3) (layer B.Cu) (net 6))
 (segment (start 117.625 45.467798) (end 125.147202 52.99) (width 0.3) (layer F.Cu) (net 6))
 (segment (start 117.625 36.2125) (end 117.625 45.467798) (width 0.3) (layer F.Cu) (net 6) (status 10))
 (segment (start 125.147202 52.99) (end 129.83 52.99) (width 0.3) (layer F.Cu) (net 6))
 (segment (start 134.92 58.08) (end 134.92 76.83) (width 0.3) (layer F.Cu) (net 6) (status 20))
 (segment (start 129.83 52.99) (end 134.92 58.08) (width 0.3) (layer F.Cu) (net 6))
 (segment (start 103.66 53.38) (end 102.71 54.33) (width 0.3) (layer B.Cu) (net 9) (status 20))
 (segment (start 107.11 53.38) (end 103.66 53.38) (width 0.3) (layer B.Cu) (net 9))
 (via (at 128.28 39.86) (size 0.8) (drill 0.4) (layers F.Cu B.Cu) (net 9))
 (segment (start 129.275 38.865) (end 129.275 36.1525) (width 0.3) (layer F.Cu) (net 9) (status 20))
 (segment (start 128.28 39.86) (end 129.275 38.865) (width 0.3) (layer F.Cu) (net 9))
 (segment (start 107.11 53.38) (end 108.45999 52.03001) (width 0.3) (layer B.Cu) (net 9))
 (segment (start 108.45999 52.03001) (end 116.10999 52.03001) (width 0.3) (layer B.Cu) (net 9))
 (segment (start 116.10999 52.03001) (end 128.28 39.86) (width 0.3) (layer B.Cu) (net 9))
 (segment (start 148.769999 78.380001) (end 150.32 76.83) (width 0.3) (layer F.Cu) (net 2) (status 20))
 (segment (start 112.420001 78.380001) (end 148.769999 78.380001) (width 0.3) (layer F.Cu) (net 2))
 (segment (start 105.4 71.36) (end 112.420001 78.380001) (width 0.3) (layer F.Cu) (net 2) (status 10))
 (segment (start 126.28 59.11) (end 129.55 62.38) (width 0.3) (layer B.Cu) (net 2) (status 10))
 (segment (start 150.32 72.37) (end 140.33 62.38) (width 0.3) (layer B.Cu) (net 2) (status 20))
 (segment (start 150.32 76.83) (end 150.32 72.37) (width 0.3) (layer B.Cu) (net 2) (status 10))
 (segment (start 117.67 30.0325) (end 129.32 30.0325) (width 0.3) (layer F.Cu) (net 2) (status 30))
 (segment (start 129.32 30.0325) (end 130.8125 30.0325) (width 0.3) (layer F.Cu) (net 2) (status 10))
 (via (at 136.87 61.38) (size 0.8) (drill 0.4) (layers F.Cu B.Cu) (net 2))
 (segment (start 136.87 55.211054) (end 136.87 61.38) (width 0.3) (layer F.Cu) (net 2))
 (segment (start 130.8125 49.153554) (end 136.87 55.211054) (width 0.3) (layer F.Cu) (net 2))
 (segment (start 130.8125 30.0325) (end 130.8125 49.153554) (width 0.3) (layer F.Cu) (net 2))
 (segment (start 137.87 62.38) (end 138.11 62.38) (width 0.3) (layer B.Cu) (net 2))
 (segment (start 136.87 61.38) (end 137.87 62.38) (width 0.3) (layer B.Cu) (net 2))
 (segment (start 138.11 62.38) (end 140.33 62.38) (width 0.3) (layer B.Cu) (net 2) (status 20))
 (segment (start 129.55 62.38) (end 138.11 62.38) (width 0.3) (layer B.Cu) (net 2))
 (segment (start 125.016399 57.833601) (end 126.28 56.57) (width 0.3) (layer B.Cu) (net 1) (status 20))
 (segment (start 118.066269 57.833601) (end 125.016399 57.833601) (width 0.3) (layer B.Cu) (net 1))
 (segment (start 116.95 58.94987) (end 118.066269 57.833601) (width 0.3) (layer B.Cu) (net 1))
 (segment (start 116.95 70.51) (end 116.95 58.94987) (width 0.3) (layer B.Cu) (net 1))
 (segment (start 113.42 74.04) (end 116.95 70.51) (width 0.3) (layer B.Cu) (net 1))
 (segment (start 100.76 74.04) (end 113.42 74.04) (width 0.3) (layer B.Cu) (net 1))
 (segment (start 99.35 72.63) (end 100.76 74.04) (width 0.3) (layer B.Cu) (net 1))
 (segment (start 99.35 70.9925) (end 99.35 72.63) (width 0.3) (layer B.Cu) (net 1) (status 10))
 (segment (start 146.63 60.08) (end 140.33 60.08) (width 0.3) (layer B.Cu) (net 3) (status 30))
 (segment (start 140.33 60.08) (end 136.37 60.08) (width 0.3) (layer B.Cu) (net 3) (status 10))
 (segment (start 136.37 60.08) (end 131.14 54.85) (width 0.3) (layer B.Cu) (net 3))
 (segment (start 125.46 54.85) (end 123.74 56.57) (width 0.3) (layer B.Cu) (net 3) (status 20))
 (segment (start 120.38 54.85) (end 125.71 54.85) (width 0.3) (layer B.Cu) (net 3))
 (segment (start 118.66 56.57) (end 120.38 54.85) (width 0.3) (layer B.Cu) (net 3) (status 10))
 (segment (start 125.71 54.85) (end 125.46 54.85) (width 0.3) (layer B.Cu) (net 3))
 (segment (start 131.14 54.85) (end 125.71 54.85) (width 0.3) (layer B.Cu) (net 3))
 (segment (start 105.0525 69.1675) (end 105.4 68.82) (width 0.3) (layer B.Cu) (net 7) (status 30))
 (segment (start 99.35 69.1675) (end 105.0525 69.1675) (width 0.3) (layer B.Cu) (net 7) (status 30))
 (segment (start 98.349999 55.232501) (end 99.36 54.2225) (width 0.3) (layer B.Cu) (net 8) (status 20))
 (segment (start 104.948934 67.069988) (end 98.349999 60.471053) (width 0.3) (layer B.Cu) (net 8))
 (segment (start 113.02 71.36) (end 108.729988 67.069988) (width 0.3) (layer B.Cu) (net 8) (status 10))
 (segment (start 108.729988 67.069988) (end 104.948934 67.069988) (width 0.3) (layer B.Cu) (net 8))
 (segment (start 98.349999 60.471053) (end 98.349999 55.232501) (width 0.3) (layer B.Cu) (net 8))
 (segment (start 139.11 46.42) (end 140.12 47.43) (width 1) (layer B.Cu) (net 5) (status 20))
 (segment (start 139.11 36.2) (end 139.11 46.42) (width 1) (layer B.Cu) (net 5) (status 10))
 (segment (start 144.11 46.42) (end 145.12 47.43) (width 1) (layer B.Cu) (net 4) (status 20))
 (segment (start 144.11 36.2) (end 144.11 46.42) (width 1) (layer B.Cu) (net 4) (status 10))
 (segment (start 101.6925 52.3975) (end 101.76 52.33) (width 0.3) (layer B.Cu) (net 10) (status 30))
 (segment (start 99.36 52.3975) (end 101.6925 52.3975) (width 0.3) (layer B.Cu) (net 10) (status 30))
 (segment (start 129.32 34.2825) (end 129.275 34.3275) (width 0.3) (layer F.Cu) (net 11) (status 30))
 (segment (start 129.32 31.9075) (end 129.32 34.2825) (width 0.3) (layer F.Cu) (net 11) (status 30))
 (segment (start 117.67 34.3425) (end 117.625 34.3875) (width 0.3) (layer F.Cu) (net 12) (status 30))
 (segment (start 117.67 31.9075) (end 117.67 34.3425) (width 0.3) (layer F.Cu) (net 12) (status 30))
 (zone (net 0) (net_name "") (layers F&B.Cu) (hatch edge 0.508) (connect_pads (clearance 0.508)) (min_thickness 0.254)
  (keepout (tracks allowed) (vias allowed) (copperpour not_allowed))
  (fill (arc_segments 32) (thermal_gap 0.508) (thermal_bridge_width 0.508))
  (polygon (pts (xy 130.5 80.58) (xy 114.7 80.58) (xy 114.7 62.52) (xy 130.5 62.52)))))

